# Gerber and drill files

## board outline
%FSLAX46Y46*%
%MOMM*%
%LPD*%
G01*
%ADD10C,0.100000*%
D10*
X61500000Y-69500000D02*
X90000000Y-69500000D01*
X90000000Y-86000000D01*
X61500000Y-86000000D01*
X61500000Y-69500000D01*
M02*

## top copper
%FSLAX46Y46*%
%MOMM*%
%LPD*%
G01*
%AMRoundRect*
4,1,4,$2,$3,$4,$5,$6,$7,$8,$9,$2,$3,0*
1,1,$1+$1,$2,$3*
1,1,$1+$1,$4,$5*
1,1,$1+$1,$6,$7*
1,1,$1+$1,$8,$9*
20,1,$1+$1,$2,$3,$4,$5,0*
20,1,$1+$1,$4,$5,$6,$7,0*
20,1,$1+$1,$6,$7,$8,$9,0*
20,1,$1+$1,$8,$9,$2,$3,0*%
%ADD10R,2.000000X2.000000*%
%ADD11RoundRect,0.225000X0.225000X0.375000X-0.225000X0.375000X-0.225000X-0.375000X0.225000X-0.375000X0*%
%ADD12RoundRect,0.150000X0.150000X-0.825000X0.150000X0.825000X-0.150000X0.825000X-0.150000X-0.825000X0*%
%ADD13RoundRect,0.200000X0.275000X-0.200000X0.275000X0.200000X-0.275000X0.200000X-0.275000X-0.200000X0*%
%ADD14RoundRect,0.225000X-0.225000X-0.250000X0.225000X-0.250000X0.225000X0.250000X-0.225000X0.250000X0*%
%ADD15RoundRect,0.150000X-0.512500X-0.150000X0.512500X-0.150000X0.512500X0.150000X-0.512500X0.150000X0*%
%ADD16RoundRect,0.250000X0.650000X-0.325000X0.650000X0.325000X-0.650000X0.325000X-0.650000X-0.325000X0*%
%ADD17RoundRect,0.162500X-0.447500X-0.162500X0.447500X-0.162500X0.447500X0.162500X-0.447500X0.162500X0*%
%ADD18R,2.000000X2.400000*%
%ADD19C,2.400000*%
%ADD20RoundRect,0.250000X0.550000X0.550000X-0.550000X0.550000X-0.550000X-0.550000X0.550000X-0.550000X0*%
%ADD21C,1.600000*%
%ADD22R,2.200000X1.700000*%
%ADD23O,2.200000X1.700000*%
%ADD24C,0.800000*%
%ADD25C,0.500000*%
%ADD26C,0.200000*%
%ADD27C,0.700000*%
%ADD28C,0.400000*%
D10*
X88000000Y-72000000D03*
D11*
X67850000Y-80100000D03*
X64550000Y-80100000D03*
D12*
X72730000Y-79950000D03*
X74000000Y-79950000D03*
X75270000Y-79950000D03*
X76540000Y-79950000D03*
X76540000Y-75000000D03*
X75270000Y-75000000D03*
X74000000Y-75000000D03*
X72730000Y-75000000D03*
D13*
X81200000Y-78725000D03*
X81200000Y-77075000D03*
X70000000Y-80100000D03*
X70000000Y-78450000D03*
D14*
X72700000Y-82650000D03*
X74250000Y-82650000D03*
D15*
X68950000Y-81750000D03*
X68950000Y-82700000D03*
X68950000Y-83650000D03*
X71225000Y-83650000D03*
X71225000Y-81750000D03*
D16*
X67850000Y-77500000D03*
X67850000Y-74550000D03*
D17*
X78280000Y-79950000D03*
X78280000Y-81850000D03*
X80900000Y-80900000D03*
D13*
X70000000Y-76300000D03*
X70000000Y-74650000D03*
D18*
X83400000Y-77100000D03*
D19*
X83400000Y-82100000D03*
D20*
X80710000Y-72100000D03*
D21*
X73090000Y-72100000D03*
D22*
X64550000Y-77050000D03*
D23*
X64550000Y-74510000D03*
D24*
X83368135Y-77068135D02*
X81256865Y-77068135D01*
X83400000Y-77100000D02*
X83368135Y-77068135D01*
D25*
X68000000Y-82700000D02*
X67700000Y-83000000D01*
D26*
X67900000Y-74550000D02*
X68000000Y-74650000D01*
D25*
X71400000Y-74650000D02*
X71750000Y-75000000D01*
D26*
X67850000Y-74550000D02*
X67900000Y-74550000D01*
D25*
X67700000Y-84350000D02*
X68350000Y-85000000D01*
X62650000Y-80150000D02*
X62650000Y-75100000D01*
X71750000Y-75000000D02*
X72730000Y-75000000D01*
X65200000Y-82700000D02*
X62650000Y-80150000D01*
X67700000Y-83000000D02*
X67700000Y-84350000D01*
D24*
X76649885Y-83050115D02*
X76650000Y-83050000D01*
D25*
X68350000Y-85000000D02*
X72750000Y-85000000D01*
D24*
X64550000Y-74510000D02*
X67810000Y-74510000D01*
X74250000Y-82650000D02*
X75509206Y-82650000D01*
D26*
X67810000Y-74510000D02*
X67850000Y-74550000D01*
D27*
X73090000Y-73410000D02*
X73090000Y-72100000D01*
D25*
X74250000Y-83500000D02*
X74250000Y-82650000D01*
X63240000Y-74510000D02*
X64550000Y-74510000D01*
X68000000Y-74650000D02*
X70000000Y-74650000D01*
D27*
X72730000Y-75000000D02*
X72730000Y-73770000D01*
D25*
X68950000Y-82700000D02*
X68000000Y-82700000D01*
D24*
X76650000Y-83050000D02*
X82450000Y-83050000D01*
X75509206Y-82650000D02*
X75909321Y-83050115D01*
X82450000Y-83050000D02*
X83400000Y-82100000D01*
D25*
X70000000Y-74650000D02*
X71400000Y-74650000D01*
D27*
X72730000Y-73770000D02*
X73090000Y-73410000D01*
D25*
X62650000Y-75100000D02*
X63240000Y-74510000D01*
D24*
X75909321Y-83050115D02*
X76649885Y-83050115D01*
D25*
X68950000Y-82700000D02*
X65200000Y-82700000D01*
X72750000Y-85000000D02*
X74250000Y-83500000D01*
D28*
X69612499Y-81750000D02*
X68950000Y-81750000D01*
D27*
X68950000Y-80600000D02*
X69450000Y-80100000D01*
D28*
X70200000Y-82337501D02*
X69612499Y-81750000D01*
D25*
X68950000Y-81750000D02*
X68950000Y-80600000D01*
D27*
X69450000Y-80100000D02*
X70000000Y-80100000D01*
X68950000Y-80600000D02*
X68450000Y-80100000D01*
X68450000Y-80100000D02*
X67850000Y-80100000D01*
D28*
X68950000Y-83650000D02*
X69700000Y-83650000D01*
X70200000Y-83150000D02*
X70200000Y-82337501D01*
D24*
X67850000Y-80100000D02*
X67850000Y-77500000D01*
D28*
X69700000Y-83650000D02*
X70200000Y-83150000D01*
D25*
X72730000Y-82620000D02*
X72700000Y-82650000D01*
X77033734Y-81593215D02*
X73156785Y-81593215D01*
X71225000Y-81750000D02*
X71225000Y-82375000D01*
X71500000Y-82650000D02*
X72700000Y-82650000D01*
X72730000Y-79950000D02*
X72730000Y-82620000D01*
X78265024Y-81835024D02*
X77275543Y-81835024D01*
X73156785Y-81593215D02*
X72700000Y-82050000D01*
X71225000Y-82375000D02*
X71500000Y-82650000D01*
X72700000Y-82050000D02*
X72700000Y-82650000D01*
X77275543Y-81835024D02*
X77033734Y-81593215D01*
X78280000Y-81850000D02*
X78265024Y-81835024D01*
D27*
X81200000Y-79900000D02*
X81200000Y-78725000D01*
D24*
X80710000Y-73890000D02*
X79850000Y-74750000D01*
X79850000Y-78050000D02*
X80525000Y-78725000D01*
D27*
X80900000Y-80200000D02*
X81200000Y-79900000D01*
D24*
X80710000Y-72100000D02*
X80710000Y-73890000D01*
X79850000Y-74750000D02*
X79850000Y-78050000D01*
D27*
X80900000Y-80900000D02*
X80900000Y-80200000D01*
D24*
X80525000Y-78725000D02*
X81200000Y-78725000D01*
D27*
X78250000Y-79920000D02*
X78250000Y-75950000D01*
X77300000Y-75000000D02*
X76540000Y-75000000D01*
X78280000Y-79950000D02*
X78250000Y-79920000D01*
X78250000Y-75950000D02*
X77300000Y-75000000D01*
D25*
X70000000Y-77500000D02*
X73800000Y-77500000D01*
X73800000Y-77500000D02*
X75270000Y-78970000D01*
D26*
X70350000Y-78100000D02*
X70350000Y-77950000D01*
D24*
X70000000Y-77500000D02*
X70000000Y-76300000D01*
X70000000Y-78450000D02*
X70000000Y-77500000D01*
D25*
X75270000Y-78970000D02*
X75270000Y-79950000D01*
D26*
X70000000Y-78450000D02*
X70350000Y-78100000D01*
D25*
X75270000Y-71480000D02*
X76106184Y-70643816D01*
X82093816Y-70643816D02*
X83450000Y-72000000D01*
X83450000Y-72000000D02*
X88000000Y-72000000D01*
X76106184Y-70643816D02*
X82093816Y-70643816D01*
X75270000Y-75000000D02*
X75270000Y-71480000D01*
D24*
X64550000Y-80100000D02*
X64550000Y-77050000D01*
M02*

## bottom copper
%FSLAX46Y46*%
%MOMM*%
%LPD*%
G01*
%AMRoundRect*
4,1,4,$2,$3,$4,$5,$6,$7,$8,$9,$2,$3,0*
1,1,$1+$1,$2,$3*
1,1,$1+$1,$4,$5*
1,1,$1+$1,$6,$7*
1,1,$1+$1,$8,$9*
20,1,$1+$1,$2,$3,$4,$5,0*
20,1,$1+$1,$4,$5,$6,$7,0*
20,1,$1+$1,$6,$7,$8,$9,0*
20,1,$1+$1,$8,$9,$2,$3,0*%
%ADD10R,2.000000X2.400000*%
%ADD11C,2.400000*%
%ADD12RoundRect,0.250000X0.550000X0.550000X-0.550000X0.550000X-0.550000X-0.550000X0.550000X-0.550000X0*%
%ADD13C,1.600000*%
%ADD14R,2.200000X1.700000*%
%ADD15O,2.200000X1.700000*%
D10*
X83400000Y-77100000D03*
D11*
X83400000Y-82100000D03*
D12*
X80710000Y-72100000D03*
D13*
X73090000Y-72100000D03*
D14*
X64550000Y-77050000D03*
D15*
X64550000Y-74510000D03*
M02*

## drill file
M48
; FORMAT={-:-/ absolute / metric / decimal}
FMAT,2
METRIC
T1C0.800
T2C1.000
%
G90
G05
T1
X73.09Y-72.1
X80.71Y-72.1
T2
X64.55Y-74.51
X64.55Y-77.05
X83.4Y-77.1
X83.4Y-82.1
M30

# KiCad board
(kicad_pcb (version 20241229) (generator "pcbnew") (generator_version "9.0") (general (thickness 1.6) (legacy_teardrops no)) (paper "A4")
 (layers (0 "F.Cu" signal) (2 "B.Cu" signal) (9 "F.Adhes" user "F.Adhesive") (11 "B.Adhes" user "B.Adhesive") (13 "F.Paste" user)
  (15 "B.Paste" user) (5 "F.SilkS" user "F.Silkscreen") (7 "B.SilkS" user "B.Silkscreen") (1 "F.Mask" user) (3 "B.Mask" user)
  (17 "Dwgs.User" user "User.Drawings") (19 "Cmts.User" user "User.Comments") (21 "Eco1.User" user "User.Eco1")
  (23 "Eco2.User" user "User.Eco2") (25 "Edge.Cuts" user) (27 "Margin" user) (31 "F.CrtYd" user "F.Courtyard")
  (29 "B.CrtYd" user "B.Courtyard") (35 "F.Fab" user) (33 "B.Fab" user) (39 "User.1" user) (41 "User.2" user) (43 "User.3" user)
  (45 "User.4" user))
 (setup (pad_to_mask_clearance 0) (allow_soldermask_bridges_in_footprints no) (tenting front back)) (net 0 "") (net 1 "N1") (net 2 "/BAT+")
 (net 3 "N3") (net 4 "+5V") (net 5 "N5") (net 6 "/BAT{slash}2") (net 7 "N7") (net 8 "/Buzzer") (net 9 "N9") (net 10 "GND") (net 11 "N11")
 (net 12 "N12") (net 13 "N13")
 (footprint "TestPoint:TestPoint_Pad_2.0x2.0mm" (layer "F.Cu") (at 88 72)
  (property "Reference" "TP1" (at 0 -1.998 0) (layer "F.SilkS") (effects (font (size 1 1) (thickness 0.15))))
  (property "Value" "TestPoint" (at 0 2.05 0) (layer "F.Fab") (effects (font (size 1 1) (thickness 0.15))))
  (pad "1" smd rect (at 0 0) (size 2 2) (layers "F.Cu" "F.Mask") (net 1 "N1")))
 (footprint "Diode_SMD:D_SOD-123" (layer "F.Cu") (at 66.2 80.1 180)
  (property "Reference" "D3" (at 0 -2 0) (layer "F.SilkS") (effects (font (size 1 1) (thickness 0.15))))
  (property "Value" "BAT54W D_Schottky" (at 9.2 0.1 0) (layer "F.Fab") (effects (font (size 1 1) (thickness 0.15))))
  (pad "1" smd roundrect (at -1.65 0 180) (size 0.9 1.2) (layers "F.Cu" "F.Mask" "F.Paste") (roundrect_rratio 0.25) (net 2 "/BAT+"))
  (pad "2" smd roundrect (at 1.65 0 180) (size 0.9 1.2) (layers "F.Cu" "F.Mask" "F.Paste") (roundrect_rratio 0.25) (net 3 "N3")))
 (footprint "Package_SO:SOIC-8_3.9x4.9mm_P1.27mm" (layer "F.Cu") (at 74.635 77.475 90)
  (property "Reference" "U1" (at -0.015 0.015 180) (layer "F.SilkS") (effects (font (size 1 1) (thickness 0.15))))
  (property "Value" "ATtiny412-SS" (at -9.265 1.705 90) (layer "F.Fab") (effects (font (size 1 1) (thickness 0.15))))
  (pad "1" smd roundrect (at -2.475 -1.905 90) (size 1.95 0.6) (layers "F.Cu" "F.Mask" "F.Paste") (roundrect_rratio 0.25) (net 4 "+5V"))
  (pad "2" smd roundrect (at -2.475 -0.635 90) (size 1.95 0.6) (layers "F.Cu" "F.Mask" "F.Paste") (roundrect_rratio 0.25) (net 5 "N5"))
  (pad "3" smd roundrect (at -2.475 0.635 90) (size 1.95 0.6) (layers "F.Cu" "F.Mask" "F.Paste") (roundrect_rratio 0.25)
   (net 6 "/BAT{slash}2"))
  (pad "4" smd roundrect (at -2.475 1.905 90) (size 1.95 0.6) (layers "F.Cu" "F.Mask" "F.Paste") (roundrect_rratio 0.25) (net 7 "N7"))
  (pad "5" smd roundrect (at 2.475 1.905 90) (size 1.95 0.6) (layers "F.Cu" "F.Mask" "F.Paste") (roundrect_rratio 0.25) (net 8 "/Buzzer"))
  (pad "6" smd roundrect (at 2.475 0.635 90) (size 1.95 0.6) (layers "F.Cu" "F.Mask" "F.Paste") (roundrect_rratio 0.25) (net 1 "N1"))
  (pad "7" smd roundrect (at 2.475 -0.635 90) (size 1.95 0.6) (layers "F.Cu" "F.Mask" "F.Paste") (roundrect_rratio 0.25) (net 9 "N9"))
  (pad "8" smd roundrect (at 2.475 -1.905 90) (size 1.95 0.6) (layers "F.Cu" "F.Mask" "F.Paste") (roundrect_rratio 0.25) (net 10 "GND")))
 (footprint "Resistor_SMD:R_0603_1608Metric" (layer "F.Cu") (at 81.2 77.9 90)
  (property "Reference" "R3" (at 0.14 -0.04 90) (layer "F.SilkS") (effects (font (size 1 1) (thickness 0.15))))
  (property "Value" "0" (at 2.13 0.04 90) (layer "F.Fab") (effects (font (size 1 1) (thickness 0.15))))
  (pad "1" smd roundrect (at -0.825 0 90) (size 0.8 0.95) (layers "F.Cu" "F.Mask" "F.Paste") (roundrect_rratio 0.25) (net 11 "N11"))
  (pad "2" smd roundrect (at 0.825 0 90) (size 0.8 0.95) (layers "F.Cu" "F.Mask" "F.Paste") (roundrect_rratio 0.25) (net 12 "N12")))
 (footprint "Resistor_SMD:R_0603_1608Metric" (layer "F.Cu") (at 70 79.275 90)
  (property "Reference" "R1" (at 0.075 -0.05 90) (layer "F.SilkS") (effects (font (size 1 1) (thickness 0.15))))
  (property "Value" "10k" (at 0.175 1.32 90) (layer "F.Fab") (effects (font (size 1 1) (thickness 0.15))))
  (pad "1" smd roundrect (at -0.825 0 90) (size 0.8 0.95) (layers "F.Cu" "F.Mask" "F.Paste") (roundrect_rratio 0.25) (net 2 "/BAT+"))
  (pad "2" smd roundrect (at 0.825 0 90) (size 0.8 0.95) (layers "F.Cu" "F.Mask" "F.Paste") (roundrect_rratio 0.25) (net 6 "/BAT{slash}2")))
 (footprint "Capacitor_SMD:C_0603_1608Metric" (layer "F.Cu") (at 73.475 82.65)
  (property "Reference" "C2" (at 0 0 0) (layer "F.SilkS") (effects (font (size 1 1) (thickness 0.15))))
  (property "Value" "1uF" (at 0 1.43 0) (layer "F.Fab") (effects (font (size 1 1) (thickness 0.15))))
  (pad "1" smd roundrect (at -0.775 0) (size 0.9 0.95) (layers "F.Cu" "F.Mask" "F.Paste") (roundrect_rratio 0.25) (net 4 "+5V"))
  (pad "2" smd roundrect (at 0.775 0) (size 0.9 0.95) (layers "F.Cu" "F.Mask" "F.Paste") (roundrect_rratio 0.25) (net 10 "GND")))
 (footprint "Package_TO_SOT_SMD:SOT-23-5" (layer "F.Cu") (at 70.0875 82.7)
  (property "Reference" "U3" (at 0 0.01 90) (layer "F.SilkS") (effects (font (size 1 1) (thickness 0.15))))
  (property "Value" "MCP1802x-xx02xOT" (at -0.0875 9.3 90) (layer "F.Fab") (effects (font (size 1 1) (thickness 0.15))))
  (pad "1" smd roundrect (at -1.1375 -0.95) (size 1.325 0.6) (layers "F.Cu" "F.Mask" "F.Paste") (roundrect_rratio 0.25) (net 2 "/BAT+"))
  (pad "2" smd roundrect (at -1.1375 0) (size 1.325 0.6) (layers "F.Cu" "F.Mask" "F.Paste") (roundrect_rratio 0.25) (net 10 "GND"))
  (pad "3" smd roundrect (at -1.1375 0.95) (size 1.325 0.6) (layers "F.Cu" "F.Mask" "F.Paste") (roundrect_rratio 0.25) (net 2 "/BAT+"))
  (pad "4" smd roundrect (at 1.1375 0.95) (size 1.325 0.6) (layers "F.Cu" "F.Mask" "F.Paste") (roundrect_rratio 0.25) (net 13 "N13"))
  (pad "5" smd roundrect (at 1.1375 -0.95) (size 1.325 0.6) (layers "F.Cu" "F.Mask" "F.Paste") (roundrect_rratio 0.25) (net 4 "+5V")))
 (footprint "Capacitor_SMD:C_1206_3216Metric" (layer "F.Cu") (at 67.85 76.025 90)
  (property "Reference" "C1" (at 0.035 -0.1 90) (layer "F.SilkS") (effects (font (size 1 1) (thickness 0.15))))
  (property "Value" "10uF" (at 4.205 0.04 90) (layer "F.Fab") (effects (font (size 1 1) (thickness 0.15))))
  (pad "1" smd roundrect (at -1.475 0 90) (size 1.15 1.8) (layers "F.Cu" "F.Mask" "F.Paste") (roundrect_rratio 0.217391) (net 2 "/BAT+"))
  (pad "2" smd roundrect (at 1.475 0 90) (size 1.15 1.8) (layers "F.Cu" "F.Mask" "F.Paste") (roundrect_rratio 0.217391) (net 10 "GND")))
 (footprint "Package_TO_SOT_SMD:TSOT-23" (layer "F.Cu") (at 79.59 80.9)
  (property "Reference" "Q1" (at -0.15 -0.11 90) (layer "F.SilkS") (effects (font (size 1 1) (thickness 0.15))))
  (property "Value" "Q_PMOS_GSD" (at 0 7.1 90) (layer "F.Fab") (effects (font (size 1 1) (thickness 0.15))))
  (pad "1" smd roundrect (at -1.31 -0.95) (size 1.22 0.65) (layers "F.Cu" "F.Mask" "F.Paste") (roundrect_rratio 0.25) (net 8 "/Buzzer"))
  (pad "2" smd roundrect (at -1.31 0.95) (size 1.22 0.65) (layers "F.Cu" "F.Mask" "F.Paste") (roundrect_rratio 0.25) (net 4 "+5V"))
  (pad "3" smd roundrect (at 1.31 0) (size 1.22 0.65) (layers "F.Cu" "F.Mask" "F.Paste") (roundrect_rratio 0.25) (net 11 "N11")))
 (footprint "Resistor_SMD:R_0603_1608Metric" (layer "F.Cu") (at 70 75.475 90)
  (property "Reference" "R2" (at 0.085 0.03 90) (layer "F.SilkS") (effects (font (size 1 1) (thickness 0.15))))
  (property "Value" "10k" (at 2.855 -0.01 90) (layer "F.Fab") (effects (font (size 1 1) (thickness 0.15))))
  (pad "1" smd roundrect (at -0.825 0 90) (size 0.8 0.95) (layers "F.Cu" "F.Mask" "F.Paste") (roundrect_rratio 0.25) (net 6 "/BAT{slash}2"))
  (pad "2" smd roundrect (at 0.825 0 90) (size 0.8 0.95) (layers "F.Cu" "F.Mask" "F.Paste") (roundrect_rratio 0.25) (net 10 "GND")))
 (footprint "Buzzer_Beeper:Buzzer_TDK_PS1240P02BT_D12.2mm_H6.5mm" (layer "B.Cu") (at 83.4 77.1 -90)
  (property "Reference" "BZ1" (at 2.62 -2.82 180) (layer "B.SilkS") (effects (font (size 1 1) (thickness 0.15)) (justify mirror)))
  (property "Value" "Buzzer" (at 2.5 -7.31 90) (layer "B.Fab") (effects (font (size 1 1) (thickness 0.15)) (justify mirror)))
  (pad "1" thru_hole rect (at 0 0 270) (size 2.4 2) (drill 1) (layers "*.Cu" "*.Mask") (remove_unused_layers no) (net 12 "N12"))
  (pad "2" thru_hole circle (at 5 0 270) (size 2.4 2.4) (drill 1) (layers "*.Cu" "*.Mask") (remove_unused_layers no) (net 10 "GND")))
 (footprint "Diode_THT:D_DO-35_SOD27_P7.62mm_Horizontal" (layer "B.Cu") (at 80.71 72.1 180)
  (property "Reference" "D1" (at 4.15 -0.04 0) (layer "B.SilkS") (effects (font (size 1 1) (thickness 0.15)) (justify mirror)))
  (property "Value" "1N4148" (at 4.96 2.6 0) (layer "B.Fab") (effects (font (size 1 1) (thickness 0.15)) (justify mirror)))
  (pad "1" thru_hole roundrect (at 0 0 180) (size 1.6 1.6) (drill 0.8) (layers "*.Cu" "*.Mask") (remove_unused_layers no)
   (roundrect_rratio 0.15625) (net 11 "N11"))
  (pad "2" thru_hole circle (at 7.62 0 180) (size 1.6 1.6) (drill 0.8) (layers "*.Cu" "*.Mask") (remove_unused_layers no) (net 10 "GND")))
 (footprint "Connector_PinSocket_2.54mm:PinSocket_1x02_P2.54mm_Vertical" (layer "B.Cu") (at 64.55 77.05)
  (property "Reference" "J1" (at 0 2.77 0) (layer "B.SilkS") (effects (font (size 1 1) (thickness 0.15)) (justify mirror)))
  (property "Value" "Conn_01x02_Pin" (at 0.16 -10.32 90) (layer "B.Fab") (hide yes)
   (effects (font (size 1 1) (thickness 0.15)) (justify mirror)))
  (pad "1" thru_hole rect (at 0 0) (size 2.2 1.7) (drill 1) (layers "*.Cu" "*.Mask") (remove_unused_layers no) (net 3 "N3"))
  (pad "2" thru_hole oval (at 0 -2.54) (size 2.2 1.7) (drill 1) (layers "*.Cu" "*.Mask") (remove_unused_layers no) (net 10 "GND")))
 (gr_rect (start 61.5 69.5) (end 90 86) (stroke (width 0.1) (type solid)) (fill no) (layer "Edge.Cuts"))
 (segment (start 83.368135 77.068135) (end 81.256865 77.068135) (width 0.8) (layer "F.Cu") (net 12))
 (segment (start 83.4 77.1) (end 83.368135 77.068135) (width 0.8) (layer "F.Cu") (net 12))
 (segment (start 68 82.7) (end 67.7 83) (width 0.5) (layer "F.Cu") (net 10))
 (segment (start 67.9 74.55) (end 68 74.65) (width 0.2) (layer "F.Cu") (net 10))
 (segment (start 71.4 74.65) (end 71.75 75) (width 0.5) (layer "F.Cu") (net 10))
 (segment (start 67.85 74.55) (end 67.9 74.55) (width 0.2) (layer "F.Cu") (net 10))
 (segment (start 67.7 84.35) (end 68.35 85) (width 0.5) (layer "F.Cu") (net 10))
 (segment (start 62.65 80.15) (end 62.65 75.1) (width 0.5) (layer "F.Cu") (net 10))
 (segment (start 71.75 75) (end 72.73 75) (width 0.5) (layer "F.Cu") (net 10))
 (segment (start 65.2 82.7) (end 62.65 80.15) (width 0.5) (layer "F.Cu") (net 10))
 (segment (start 67.7 83) (end 67.7 84.35) (width 0.5) (layer "F.Cu") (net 10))
 (segment (start 76.649885 83.050115) (end 76.65 83.05) (width 0.8) (layer "F.Cu") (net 10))
 (segment (start 68.35 85) (end 72.75 85) (width 0.5) (layer "F.Cu") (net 10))
 (segment (start 64.55 74.51) (end 67.81 74.51) (width 0.8) (layer "F.Cu") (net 10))
 (segment (start 74.25 82.65) (end 75.509206 82.65) (width 0.8) (layer "F.Cu") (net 10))
 (segment (start 67.81 74.51) (end 67.85 74.55) (width 0.2) (layer "F.Cu") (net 10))
 (segment (start 73.09 73.41) (end 73.09 72.1) (width 0.7) (layer "F.Cu") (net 10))
 (segment (start 74.25 83.5) (end 74.25 82.65) (width 0.5) (layer "F.Cu") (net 10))
 (segment (start 63.24 74.51) (end 64.55 74.51) (width 0.5) (layer "F.Cu") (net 10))
 (segment (start 68 74.65) (end 70 74.65) (width 0.5) (layer "F.Cu") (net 10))
 (segment (start 72.73 75) (end 72.73 73.77) (width 0.7) (layer "F.Cu") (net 10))
 (segment (start 68.95 82.7) (end 68 82.7) (width 0.5) (layer "F.Cu") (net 10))
 (segment (start 76.65 83.05) (end 82.45 83.05) (width 0.8) (layer "F.Cu") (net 10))
 (segment (start 75.509206 82.65) (end 75.909321 83.050115) (width 0.8) (layer "F.Cu") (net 10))
 (segment (start 82.45 83.05) (end 83.4 82.1) (width 0.8) (layer "F.Cu") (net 10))
 (segment (start 70 74.65) (end 71.4 74.65) (width 0.5) (layer "F.Cu") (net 10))
 (segment (start 72.73 73.77) (end 73.09 73.41) (width 0.7) (layer "F.Cu") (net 10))
 (segment (start 62.65 75.1) (end 63.24 74.51) (width 0.5) (layer "F.Cu") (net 10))
 (segment (start 75.909321 83.050115) (end 76.649885 83.050115) (width 0.8) (layer "F.Cu") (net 10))
 (segment (start 68.95 82.7) (end 65.2 82.7) (width 0.5) (layer "F.Cu") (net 10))
 (segment (start 72.75 85) (end 74.25 83.5) (width 0.5) (layer "F.Cu") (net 10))
 (segment (start 69.612499 81.75) (end 68.95 81.75) (width 0.4) (layer "F.Cu") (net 2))
 (segment (start 68.95 80.6) (end 69.45 80.1) (width 0.7) (layer "F.Cu") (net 2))
 (segment (start 70.2 82.337501) (end 69.612499 81.75) (width 0.4) (layer "F.Cu") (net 2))
 (segment (start 68.95 81.75) (end 68.95 80.6) (width 0.5) (layer "F.Cu") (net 2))
 (segment (start 69.45 80.1) (end 70 80.1) (width 0.7) (layer "F.Cu") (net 2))
 (segment (start 68.95 80.6) (end 68.45 80.1) (width 0.7) (layer "F.Cu") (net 2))
 (segment (start 68.45 80.1) (end 67.85 80.1) (width 0.7) (layer "F.Cu") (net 2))
 (segment (start 68.95 83.65) (end 69.7 83.65) (width 0.4) (layer "F.Cu") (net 2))
 (segment (start 70.2 83.15) (end 70.2 82.337501) (width 0.4) (layer "F.Cu") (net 2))
 (segment (start 67.85 80.1) (end 67.85 77.5) (width 0.8) (layer "F.Cu") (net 2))
 (segment (start 69.7 83.65) (end 70.2 83.15) (width 0.4) (layer "F.Cu") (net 2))
 (segment (start 72.73 82.62) (end 72.7 82.65) (width 0.5) (layer "F.Cu") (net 4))
 (segment (start 77.033734 81.593215) (end 73.156785 81.593215) (width 0.5) (layer "F.Cu") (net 4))
 (segment (start 71.225 81.75) (end 71.225 82.375) (width 0.5) (layer "F.Cu") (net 4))
 (segment (start 71.5 82.65) (end 72.7 82.65) (width 0.5) (layer "F.Cu") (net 4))
 (segment (start 72.73 79.95) (end 72.73 82.62) (width 0.5) (layer "F.Cu") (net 4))
 (segment (start 78.265024 81.835024) (end 77.275543 81.835024) (width 0.5) (layer "F.Cu") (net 4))
 (segment (start 73.156785 81.593215) (end 72.7 82.05) (width 0.5) (layer "F.Cu") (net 4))
 (segment (start 71.225 82.375) (end 71.5 82.65) (width 0.5) (layer "F.Cu") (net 4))
 (segment (start 72.7 82.05) (end 72.7 82.65) (width 0.5) (layer "F.Cu") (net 4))
 (segment (start 77.275543 81.835024) (end 77.033734 81.593215) (width 0.5) (layer "F.Cu") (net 4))
 (segment (start 78.28 81.85) (end 78.265024 81.835024) (width 0.5) (layer "F.Cu") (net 4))
 (segment (start 81.2 79.9) (end 81.2 78.725) (width 0.7) (layer "F.Cu") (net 11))
 (segment (start 80.71 73.89) (end 79.85 74.75) (width 0.8) (layer "F.Cu") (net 11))
 (segment (start 79.85 78.05) (end 80.525 78.725) (width 0.8) (layer "F.Cu") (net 11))
 (segment (start 80.9 80.2) (end 81.2 79.9) (width 0.7) (layer "F.Cu") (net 11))
 (segment (start 80.71 72.1) (end 80.71 73.89) (width 0.8) (layer "F.Cu") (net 11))
 (segment (start 79.85 74.75) (end 79.85 78.05) (width 0.8) (layer "F.Cu") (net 11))
 (segment (start 80.9 80.9) (end 80.9 80.2) (width 0.7) (layer "F.Cu") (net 11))
 (segment (start 80.525 78.725) (end 81.2 78.725) (width 0.8) (layer "F.Cu") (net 11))
 (segment (start 78.25 79.92) (end 78.25 75.95) (width 0.7) (layer "F.Cu") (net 8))
 (segment (start 77.3 75) (end 76.54 75) (width 0.7) (layer "F.Cu") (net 8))
 (segment (start 78.28 79.95) (end 78.25 79.92) (width 0.7) (layer "F.Cu") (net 8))
 (segment (start 78.25 75.95) (end 77.3 75) (width 0.7) (layer "F.Cu") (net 8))
 (segment (start 70 77.5) (end 73.8 77.5) (width 0.5) (layer "F.Cu") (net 6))
 (segment (start 73.8 77.5) (end 75.27 78.97) (width 0.5) (layer "F.Cu") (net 6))
 (segment (start 70.35 78.1) (end 70.35 77.95) (width 0.2) (layer "F.Cu") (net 6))
 (segment (start 70 77.5) (end 70 76.3) (width 0.8) (layer "F.Cu") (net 6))
 (segment (start 70 78.45) (end 70 77.5) (width 0.8) (layer "F.Cu") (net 6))
 (segment (start 75.27 78.97) (end 75.27 79.95) (width 0.5) (layer "F.Cu") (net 6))
 (segment (start 70 78.45) (end 70.35 78.1) (width 0.2) (layer "F.Cu") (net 6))
 (segment (start 75.27 71.48) (end 76.106184 70.643816) (width 0.5) (layer "F.Cu") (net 1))
 (segment (start 82.093816 70.643816) (end 83.45 72) (width 0.5) (layer "F.Cu") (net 1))
 (segment (start 83.45 72) (end 88 72) (width 0.5) (layer "F.Cu") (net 1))
 (segment (start 76.106184 70.643816) (end 82.093816 70.643816) (width 0.5) (layer "F.Cu") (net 1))
 (segment (start 75.27 75) (end 75.27 71.48) (width 0.5) (layer "F.Cu") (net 1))
 (segment (start 64.55 80.1) (end 64.55 77.05) (width 0.8) (layer "F.Cu") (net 3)))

